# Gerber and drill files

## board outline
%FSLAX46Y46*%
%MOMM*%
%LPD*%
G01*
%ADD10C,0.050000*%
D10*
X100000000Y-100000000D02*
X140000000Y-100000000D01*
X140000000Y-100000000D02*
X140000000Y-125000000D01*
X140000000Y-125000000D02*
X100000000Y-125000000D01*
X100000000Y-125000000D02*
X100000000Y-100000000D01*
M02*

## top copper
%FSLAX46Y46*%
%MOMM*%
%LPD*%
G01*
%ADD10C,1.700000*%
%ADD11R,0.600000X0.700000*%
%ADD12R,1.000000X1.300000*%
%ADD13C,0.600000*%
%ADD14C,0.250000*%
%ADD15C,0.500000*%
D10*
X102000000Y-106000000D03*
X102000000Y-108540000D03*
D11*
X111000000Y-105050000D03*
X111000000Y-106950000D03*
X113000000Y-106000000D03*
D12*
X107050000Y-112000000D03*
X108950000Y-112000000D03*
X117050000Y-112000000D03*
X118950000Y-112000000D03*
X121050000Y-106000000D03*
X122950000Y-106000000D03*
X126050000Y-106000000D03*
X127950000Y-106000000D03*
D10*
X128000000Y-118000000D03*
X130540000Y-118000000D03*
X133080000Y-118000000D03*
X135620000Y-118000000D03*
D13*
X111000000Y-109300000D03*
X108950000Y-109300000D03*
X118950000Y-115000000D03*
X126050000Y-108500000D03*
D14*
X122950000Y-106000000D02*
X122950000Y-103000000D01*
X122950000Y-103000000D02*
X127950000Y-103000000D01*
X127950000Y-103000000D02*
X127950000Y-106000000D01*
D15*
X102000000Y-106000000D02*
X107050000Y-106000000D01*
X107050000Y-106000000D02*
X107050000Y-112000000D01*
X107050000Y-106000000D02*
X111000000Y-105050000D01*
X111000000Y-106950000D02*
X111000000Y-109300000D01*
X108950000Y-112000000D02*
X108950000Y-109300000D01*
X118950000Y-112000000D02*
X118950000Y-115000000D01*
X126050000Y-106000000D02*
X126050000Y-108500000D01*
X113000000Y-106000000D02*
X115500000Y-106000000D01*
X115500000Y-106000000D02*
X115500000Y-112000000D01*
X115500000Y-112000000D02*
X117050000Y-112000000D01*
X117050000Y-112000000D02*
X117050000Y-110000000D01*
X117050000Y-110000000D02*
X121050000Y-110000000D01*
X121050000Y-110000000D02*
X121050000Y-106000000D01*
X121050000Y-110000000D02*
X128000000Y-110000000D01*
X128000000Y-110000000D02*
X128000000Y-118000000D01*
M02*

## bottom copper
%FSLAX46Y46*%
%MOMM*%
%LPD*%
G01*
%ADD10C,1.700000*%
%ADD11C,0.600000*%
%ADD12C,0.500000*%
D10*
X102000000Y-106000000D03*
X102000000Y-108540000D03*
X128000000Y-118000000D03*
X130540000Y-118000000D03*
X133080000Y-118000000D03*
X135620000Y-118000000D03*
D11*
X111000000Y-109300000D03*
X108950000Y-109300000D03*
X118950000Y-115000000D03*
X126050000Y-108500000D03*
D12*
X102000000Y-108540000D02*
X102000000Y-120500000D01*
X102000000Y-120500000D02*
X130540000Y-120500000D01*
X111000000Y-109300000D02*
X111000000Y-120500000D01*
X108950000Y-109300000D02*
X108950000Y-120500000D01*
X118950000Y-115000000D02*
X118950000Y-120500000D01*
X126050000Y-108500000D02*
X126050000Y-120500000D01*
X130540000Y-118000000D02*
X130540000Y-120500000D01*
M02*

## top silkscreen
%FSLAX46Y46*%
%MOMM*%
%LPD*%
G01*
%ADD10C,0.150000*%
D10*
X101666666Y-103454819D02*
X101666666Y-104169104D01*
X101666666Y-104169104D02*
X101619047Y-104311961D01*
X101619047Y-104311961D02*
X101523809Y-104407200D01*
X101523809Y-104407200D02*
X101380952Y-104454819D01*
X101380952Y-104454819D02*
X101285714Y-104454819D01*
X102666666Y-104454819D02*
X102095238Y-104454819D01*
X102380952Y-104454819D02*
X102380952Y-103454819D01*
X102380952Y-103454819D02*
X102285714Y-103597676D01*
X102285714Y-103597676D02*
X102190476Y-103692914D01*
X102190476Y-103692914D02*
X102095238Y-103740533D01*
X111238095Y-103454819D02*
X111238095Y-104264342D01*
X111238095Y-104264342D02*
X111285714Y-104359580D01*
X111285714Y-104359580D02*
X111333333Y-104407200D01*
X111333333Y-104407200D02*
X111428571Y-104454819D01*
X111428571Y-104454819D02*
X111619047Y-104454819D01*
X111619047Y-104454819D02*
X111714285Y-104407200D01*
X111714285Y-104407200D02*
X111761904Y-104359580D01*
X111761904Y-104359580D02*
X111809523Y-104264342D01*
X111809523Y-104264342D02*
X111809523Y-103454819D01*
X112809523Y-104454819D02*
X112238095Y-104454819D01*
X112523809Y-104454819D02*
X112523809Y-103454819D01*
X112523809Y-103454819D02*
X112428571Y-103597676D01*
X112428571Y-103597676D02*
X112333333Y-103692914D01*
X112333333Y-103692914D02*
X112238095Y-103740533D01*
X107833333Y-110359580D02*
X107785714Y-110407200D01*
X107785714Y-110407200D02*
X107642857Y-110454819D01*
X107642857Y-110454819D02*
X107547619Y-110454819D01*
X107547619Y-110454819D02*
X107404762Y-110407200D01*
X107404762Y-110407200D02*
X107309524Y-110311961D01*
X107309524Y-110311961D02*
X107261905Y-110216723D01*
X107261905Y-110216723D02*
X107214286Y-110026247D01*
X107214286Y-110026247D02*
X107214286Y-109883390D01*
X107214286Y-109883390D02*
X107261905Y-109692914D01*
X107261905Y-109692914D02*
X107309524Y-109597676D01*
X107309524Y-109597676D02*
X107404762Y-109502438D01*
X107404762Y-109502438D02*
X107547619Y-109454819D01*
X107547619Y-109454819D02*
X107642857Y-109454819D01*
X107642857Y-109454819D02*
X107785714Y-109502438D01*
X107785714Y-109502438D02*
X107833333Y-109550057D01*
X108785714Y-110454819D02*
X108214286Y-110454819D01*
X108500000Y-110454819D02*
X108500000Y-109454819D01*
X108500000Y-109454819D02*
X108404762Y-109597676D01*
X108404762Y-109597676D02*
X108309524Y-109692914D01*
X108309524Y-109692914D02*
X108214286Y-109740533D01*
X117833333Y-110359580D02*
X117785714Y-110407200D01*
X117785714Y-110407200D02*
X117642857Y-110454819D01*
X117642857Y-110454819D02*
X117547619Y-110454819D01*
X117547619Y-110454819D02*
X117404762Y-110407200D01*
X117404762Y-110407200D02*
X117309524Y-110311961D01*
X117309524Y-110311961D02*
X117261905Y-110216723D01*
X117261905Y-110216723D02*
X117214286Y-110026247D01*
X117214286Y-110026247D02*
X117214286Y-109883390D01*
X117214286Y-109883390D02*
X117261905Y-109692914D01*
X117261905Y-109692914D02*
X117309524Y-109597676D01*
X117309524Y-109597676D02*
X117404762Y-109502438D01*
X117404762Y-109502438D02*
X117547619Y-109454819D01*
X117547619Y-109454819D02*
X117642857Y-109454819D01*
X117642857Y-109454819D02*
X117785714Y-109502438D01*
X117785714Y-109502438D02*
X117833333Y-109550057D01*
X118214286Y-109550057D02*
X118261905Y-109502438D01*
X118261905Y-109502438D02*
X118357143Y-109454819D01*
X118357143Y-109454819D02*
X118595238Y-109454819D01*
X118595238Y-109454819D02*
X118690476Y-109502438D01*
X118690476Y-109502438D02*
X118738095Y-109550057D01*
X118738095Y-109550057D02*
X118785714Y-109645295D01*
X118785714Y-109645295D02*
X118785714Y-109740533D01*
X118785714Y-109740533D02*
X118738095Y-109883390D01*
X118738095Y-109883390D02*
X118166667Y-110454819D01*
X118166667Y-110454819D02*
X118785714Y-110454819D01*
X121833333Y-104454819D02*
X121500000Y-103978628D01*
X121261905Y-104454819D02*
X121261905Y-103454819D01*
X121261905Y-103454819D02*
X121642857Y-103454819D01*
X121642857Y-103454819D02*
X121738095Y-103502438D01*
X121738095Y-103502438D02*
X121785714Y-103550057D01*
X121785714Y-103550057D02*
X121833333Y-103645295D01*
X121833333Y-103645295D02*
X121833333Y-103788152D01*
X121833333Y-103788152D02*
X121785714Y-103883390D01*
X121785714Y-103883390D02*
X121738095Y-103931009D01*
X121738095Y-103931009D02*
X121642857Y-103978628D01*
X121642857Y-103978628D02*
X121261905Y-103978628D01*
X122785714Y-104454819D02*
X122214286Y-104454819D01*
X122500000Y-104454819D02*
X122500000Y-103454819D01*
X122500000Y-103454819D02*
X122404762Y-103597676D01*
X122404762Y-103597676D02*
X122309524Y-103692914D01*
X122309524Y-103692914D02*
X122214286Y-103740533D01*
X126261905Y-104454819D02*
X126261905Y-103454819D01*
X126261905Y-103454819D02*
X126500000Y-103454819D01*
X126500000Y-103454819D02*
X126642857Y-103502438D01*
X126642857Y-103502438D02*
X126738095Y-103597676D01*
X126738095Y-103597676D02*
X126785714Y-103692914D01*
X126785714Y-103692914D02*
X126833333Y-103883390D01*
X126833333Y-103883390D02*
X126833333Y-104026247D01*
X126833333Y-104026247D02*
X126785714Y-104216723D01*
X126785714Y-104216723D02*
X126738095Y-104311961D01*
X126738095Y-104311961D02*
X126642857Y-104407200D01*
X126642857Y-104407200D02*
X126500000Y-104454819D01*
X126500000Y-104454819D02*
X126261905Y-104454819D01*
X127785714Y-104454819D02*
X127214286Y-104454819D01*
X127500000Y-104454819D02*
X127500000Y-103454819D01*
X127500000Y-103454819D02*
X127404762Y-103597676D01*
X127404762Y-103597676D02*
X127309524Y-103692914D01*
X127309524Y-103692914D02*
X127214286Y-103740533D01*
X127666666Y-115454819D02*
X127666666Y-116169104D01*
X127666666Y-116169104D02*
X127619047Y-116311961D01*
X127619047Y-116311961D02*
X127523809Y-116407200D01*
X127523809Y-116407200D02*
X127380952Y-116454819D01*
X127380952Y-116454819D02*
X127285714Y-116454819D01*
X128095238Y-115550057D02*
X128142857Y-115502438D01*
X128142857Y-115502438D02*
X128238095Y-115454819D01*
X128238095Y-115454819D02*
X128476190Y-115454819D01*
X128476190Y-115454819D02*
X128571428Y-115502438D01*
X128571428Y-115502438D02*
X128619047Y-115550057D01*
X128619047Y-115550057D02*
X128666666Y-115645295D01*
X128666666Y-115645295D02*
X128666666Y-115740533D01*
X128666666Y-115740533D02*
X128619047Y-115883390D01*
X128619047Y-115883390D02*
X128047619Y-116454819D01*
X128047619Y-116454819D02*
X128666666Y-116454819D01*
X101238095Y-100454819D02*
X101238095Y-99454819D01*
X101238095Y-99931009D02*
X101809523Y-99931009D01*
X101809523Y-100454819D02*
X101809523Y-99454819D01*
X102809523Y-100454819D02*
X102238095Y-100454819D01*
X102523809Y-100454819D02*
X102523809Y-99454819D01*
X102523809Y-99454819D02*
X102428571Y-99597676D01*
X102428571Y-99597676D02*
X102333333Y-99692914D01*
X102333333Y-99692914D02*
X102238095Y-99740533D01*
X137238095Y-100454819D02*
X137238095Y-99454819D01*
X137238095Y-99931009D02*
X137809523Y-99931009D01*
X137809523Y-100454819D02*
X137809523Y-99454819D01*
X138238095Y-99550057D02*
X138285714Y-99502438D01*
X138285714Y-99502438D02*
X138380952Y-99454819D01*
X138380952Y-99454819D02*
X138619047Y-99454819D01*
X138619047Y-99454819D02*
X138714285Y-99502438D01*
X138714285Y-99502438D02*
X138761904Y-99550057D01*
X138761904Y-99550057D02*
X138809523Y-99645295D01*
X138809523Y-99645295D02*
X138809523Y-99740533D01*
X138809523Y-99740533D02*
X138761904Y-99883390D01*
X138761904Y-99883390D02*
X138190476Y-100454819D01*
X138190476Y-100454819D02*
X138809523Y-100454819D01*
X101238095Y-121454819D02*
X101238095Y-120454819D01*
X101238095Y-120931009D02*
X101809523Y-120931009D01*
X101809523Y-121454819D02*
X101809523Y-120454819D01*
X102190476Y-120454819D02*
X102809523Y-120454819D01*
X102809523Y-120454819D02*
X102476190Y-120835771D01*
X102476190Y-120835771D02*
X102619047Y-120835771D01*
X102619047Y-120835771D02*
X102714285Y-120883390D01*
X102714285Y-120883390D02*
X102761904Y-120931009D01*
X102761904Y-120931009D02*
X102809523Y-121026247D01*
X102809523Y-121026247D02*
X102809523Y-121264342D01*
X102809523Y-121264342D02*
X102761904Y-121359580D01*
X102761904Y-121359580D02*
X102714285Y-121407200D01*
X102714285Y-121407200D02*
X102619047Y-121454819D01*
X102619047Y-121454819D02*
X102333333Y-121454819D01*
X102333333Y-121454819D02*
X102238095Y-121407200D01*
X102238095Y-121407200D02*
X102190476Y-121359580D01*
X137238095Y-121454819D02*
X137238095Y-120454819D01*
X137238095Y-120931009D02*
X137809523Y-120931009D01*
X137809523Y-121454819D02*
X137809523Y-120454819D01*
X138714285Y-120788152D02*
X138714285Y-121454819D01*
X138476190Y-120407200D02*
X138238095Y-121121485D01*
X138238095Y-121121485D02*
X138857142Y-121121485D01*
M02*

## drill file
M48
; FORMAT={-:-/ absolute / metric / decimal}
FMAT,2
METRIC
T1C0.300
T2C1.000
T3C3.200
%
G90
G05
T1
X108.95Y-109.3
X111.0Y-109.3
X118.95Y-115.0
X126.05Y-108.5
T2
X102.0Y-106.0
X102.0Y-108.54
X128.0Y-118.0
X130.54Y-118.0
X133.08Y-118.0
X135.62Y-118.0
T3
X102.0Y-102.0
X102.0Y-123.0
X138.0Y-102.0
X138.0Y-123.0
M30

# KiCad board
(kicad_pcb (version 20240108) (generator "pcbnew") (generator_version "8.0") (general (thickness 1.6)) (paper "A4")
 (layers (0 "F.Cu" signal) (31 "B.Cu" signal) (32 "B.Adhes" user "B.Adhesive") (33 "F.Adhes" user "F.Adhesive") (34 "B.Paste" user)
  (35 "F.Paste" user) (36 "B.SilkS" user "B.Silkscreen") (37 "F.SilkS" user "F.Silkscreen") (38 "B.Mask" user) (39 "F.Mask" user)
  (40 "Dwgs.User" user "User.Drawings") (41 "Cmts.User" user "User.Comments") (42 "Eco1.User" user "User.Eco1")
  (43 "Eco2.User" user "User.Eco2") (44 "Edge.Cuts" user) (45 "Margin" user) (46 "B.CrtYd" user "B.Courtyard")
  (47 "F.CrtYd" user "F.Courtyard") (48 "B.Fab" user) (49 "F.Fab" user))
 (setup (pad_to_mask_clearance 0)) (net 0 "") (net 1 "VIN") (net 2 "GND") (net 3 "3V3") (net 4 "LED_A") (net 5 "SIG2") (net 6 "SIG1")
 (gr_line (start 100 100) (end 140 100) (stroke (width 0.05) (type default)) (layer "Edge.Cuts"))
 (gr_line (start 140 100) (end 140 125) (stroke (width 0.05) (type default)) (layer "Edge.Cuts"))
 (gr_line (start 140 125) (end 100 125) (stroke (width 0.05) (type default)) (layer "Edge.Cuts"))
 (gr_line (start 100 125) (end 100 100) (stroke (width 0.05) (type default)) (layer "Edge.Cuts"))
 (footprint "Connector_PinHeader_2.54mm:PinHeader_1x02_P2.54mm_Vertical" (layer "F.Cu") (at 102 106)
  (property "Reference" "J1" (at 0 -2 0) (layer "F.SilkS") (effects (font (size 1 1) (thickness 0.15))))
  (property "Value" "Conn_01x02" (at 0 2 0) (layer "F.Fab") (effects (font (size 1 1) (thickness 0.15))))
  (pad "1" thru_hole circle (at 0 0) (size 1.7 1.7) (drill 1) (layers "*.Cu" "*.Mask") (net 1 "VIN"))
  (pad "2" thru_hole circle (at 0 2.54) (size 1.7 1.7) (drill 1) (layers "*.Cu" "*.Mask") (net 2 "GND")))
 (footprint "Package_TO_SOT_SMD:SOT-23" (layer "F.Cu") (at 112 106)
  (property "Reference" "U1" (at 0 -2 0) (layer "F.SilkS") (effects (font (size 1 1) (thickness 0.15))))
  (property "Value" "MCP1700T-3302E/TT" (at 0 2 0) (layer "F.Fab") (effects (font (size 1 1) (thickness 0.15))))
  (pad "1" smd rect (at -1 -0.95) (size 0.6 0.7) (layers "F.Cu" "F.Paste" "F.Mask") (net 1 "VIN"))
  (pad "2" smd rect (at -1 0.95) (size 0.6 0.7) (layers "F.Cu" "F.Paste" "F.Mask") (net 2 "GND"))
  (pad "3" smd rect (at 1 0) (size 0.6 0.7) (layers "F.Cu" "F.Paste" "F.Mask") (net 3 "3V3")))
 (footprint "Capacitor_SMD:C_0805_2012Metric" (layer "F.Cu") (at 108 112)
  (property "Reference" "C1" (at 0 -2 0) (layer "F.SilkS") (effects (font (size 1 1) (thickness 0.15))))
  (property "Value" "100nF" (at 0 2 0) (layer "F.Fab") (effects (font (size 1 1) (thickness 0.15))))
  (pad "1" smd rect (at -0.95 0) (size 1 1.3) (layers "F.Cu" "F.Paste" "F.Mask") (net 1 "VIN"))
  (pad "2" smd rect (at 0.95 0) (size 1 1.3) (layers "F.Cu" "F.Paste" "F.Mask") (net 2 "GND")))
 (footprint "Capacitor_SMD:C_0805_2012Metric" (layer "F.Cu") (at 118 112)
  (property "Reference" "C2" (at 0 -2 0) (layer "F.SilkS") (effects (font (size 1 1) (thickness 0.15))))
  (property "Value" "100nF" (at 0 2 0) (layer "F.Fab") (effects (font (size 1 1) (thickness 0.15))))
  (pad "1" smd rect (at -0.95 0) (size 1 1.3) (layers "F.Cu" "F.Paste" "F.Mask") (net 3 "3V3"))
  (pad "2" smd rect (at 0.95 0) (size 1 1.3) (layers "F.Cu" "F.Paste" "F.Mask") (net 2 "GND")))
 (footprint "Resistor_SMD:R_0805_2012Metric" (layer "F.Cu") (at 122 106)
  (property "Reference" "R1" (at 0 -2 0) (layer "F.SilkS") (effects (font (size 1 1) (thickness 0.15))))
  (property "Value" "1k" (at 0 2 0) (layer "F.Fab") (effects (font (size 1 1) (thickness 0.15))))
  (pad "1" smd rect (at -0.95 0) (size 1 1.3) (layers "F.Cu" "F.Paste" "F.Mask") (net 3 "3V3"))
  (pad "2" smd rect (at 0.95 0) (size 1 1.3) (layers "F.Cu" "F.Paste" "F.Mask") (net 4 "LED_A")))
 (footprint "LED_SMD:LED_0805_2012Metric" (layer "F.Cu") (at 127 106)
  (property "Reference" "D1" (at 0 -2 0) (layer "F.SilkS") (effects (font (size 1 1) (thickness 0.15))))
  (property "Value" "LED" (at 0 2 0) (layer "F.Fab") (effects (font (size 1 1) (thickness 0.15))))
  (pad "1" smd rect (at -0.95 0) (size 1 1.3) (layers "F.Cu" "F.Paste" "F.Mask") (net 2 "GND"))
  (pad "2" smd rect (at 0.95 0) (size 1 1.3) (layers "F.Cu" "F.Paste" "F.Mask") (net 4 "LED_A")))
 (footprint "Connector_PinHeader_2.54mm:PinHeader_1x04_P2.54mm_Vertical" (layer "F.Cu") (at 128 118)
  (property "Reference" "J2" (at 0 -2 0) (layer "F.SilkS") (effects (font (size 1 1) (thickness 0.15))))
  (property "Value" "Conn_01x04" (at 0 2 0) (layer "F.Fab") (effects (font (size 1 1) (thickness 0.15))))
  (pad "1" thru_hole circle (at 0 0) (size 1.7 1.7) (drill 1) (layers "*.Cu" "*.Mask") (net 3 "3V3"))
  (pad "2" thru_hole circle (at 2.54 0) (size 1.7 1.7) (drill 1) (layers "*.Cu" "*.Mask") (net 2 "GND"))
  (pad "3" thru_hole circle (at 5.08 0) (size 1.7 1.7) (drill 1) (layers "*.Cu" "*.Mask") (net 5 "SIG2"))
  (pad "4" thru_hole circle (at 7.62 0) (size 1.7 1.7) (drill 1) (layers "*.Cu" "*.Mask") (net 5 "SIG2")))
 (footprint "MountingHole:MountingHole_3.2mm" (layer "F.Cu") (at 102 102)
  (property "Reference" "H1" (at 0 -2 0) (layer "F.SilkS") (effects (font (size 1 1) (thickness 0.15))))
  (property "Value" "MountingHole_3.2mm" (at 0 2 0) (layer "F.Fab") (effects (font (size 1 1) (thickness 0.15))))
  (pad "1" np_thru_hole circle (at 0 0) (size 3.2 3.2) (drill 3.2) (layers "*.Cu" "*.Mask")))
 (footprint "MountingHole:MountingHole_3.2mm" (layer "F.Cu") (at 138 102)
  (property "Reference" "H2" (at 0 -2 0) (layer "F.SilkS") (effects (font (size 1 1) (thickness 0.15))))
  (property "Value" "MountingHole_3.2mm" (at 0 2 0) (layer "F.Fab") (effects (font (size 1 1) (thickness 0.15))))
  (pad "1" np_thru_hole circle (at 0 0) (size 3.2 3.2) (drill 3.2) (layers "*.Cu" "*.Mask")))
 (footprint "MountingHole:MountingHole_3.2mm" (layer "F.Cu") (at 102 123)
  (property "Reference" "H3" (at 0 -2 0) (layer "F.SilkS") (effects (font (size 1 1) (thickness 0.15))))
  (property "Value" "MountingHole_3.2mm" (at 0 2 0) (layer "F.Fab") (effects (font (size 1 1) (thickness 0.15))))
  (pad "1" np_thru_hole circle (at 0 0) (size 3.2 3.2) (drill 3.2) (layers "*.Cu" "*.Mask")))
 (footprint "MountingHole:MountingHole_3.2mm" (layer "F.Cu") (at 138 123)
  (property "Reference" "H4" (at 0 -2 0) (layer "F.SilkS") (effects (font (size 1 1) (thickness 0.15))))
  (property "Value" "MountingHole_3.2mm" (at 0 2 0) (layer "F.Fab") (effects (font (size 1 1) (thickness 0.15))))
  (pad "1" np_thru_hole circle (at 0 0) (size 3.2 3.2) (drill 3.2) (layers "*.Cu" "*.Mask")))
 (segment (start 122.95 106) (end 122.95 103) (width 0.25) (layer "F.Cu") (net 4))
 (segment (start 122.95 103) (end 127.95 103) (width 0.25) (layer "F.Cu") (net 4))
 (segment (start 127.95 103) (end 127.95 106) (width 0.25) (layer "F.Cu") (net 4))
 (segment (start 102 106) (end 107.05 106) (width 0.5) (layer "F.Cu") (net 1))
 (segment (start 107.05 106) (end 107.05 112) (width 0.5) (layer "F.Cu") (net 1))
 (segment (start 107.05 106) (end 111 105.05) (width 0.5) (layer "F.Cu") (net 1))
 (segment (start 111 106.95) (end 111 109.3) (width 0.5) (layer "F.Cu") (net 2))
 (segment (start 108.95 112) (end 108.95 109.3) (width 0.5) (layer "F.Cu") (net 2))
 (segment (start 118.95 112) (end 118.95 115) (width 0.5) (layer "F.Cu") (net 2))
 (segment (start 126.05 106) (end 126.05 108.5) (width 0.5) (layer "F.Cu") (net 2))
 (segment (start 113 106) (end 115.5 106) (width 0.5) (layer "F.Cu") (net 3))
 (segment (start 115.5 106) (end 115.5 112) (width 0.5) (layer "F.Cu") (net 3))
 (segment (start 115.5 112) (end 117.05 112) (width 0.5) (layer "F.Cu") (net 3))
 (segment (start 117.05 112) (end 117.05 110) (width 0.5) (layer "F.Cu") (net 3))
 (segment (start 117.05 110) (end 121.05 110) (width 0.5) (layer "F.Cu") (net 3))
 (segment (start 121.05 110) (end 121.05 106) (width 0.5) (layer "F.Cu") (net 3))
 (segment (start 121.05 110) (end 128 110) (width 0.5) (layer "F.Cu") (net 3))
 (segment (start 128 110) (end 128 118) (width 0.5) (layer "F.Cu") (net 3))
 (segment (start 102 108.54) (end 102 120.5) (width 0.5) (layer "B.Cu") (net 2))
 (segment (start 102 120.5) (end 130.54 120.5) (width 0.5) (layer "B.Cu") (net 2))
 (segment (start 111 109.3) (end 111 120.5) (width 0.5) (layer "B.Cu") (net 2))
 (segment (start 108.95 109.3) (end 108.95 120.5) (width 0.5) (layer "B.Cu") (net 2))
 (segment (start 118.95 115) (end 118.95 120.5) (width 0.5) (layer "B.Cu") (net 2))
 (segment (start 126.05 108.5) (end 126.05 120.5) (width 0.5) (layer "B.Cu") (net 2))
 (segment (start 130.54 118) (end 130.54 120.5) (width 0.5) (layer "B.Cu") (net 2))
 (via (at 111 109.3) (size 0.6) (drill 0.3) (layers "F.Cu" "B.Cu") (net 2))
 (via (at 108.95 109.3) (size 0.6) (drill 0.3) (layers "F.Cu" "B.Cu") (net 2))
 (via (at 118.95 115) (size 0.6) (drill 0.3) (layers "F.Cu" "B.Cu") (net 2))
 (via (at 126.05 108.5) (size 0.6) (drill 0.3) (layers "F.Cu" "B.Cu") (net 2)))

